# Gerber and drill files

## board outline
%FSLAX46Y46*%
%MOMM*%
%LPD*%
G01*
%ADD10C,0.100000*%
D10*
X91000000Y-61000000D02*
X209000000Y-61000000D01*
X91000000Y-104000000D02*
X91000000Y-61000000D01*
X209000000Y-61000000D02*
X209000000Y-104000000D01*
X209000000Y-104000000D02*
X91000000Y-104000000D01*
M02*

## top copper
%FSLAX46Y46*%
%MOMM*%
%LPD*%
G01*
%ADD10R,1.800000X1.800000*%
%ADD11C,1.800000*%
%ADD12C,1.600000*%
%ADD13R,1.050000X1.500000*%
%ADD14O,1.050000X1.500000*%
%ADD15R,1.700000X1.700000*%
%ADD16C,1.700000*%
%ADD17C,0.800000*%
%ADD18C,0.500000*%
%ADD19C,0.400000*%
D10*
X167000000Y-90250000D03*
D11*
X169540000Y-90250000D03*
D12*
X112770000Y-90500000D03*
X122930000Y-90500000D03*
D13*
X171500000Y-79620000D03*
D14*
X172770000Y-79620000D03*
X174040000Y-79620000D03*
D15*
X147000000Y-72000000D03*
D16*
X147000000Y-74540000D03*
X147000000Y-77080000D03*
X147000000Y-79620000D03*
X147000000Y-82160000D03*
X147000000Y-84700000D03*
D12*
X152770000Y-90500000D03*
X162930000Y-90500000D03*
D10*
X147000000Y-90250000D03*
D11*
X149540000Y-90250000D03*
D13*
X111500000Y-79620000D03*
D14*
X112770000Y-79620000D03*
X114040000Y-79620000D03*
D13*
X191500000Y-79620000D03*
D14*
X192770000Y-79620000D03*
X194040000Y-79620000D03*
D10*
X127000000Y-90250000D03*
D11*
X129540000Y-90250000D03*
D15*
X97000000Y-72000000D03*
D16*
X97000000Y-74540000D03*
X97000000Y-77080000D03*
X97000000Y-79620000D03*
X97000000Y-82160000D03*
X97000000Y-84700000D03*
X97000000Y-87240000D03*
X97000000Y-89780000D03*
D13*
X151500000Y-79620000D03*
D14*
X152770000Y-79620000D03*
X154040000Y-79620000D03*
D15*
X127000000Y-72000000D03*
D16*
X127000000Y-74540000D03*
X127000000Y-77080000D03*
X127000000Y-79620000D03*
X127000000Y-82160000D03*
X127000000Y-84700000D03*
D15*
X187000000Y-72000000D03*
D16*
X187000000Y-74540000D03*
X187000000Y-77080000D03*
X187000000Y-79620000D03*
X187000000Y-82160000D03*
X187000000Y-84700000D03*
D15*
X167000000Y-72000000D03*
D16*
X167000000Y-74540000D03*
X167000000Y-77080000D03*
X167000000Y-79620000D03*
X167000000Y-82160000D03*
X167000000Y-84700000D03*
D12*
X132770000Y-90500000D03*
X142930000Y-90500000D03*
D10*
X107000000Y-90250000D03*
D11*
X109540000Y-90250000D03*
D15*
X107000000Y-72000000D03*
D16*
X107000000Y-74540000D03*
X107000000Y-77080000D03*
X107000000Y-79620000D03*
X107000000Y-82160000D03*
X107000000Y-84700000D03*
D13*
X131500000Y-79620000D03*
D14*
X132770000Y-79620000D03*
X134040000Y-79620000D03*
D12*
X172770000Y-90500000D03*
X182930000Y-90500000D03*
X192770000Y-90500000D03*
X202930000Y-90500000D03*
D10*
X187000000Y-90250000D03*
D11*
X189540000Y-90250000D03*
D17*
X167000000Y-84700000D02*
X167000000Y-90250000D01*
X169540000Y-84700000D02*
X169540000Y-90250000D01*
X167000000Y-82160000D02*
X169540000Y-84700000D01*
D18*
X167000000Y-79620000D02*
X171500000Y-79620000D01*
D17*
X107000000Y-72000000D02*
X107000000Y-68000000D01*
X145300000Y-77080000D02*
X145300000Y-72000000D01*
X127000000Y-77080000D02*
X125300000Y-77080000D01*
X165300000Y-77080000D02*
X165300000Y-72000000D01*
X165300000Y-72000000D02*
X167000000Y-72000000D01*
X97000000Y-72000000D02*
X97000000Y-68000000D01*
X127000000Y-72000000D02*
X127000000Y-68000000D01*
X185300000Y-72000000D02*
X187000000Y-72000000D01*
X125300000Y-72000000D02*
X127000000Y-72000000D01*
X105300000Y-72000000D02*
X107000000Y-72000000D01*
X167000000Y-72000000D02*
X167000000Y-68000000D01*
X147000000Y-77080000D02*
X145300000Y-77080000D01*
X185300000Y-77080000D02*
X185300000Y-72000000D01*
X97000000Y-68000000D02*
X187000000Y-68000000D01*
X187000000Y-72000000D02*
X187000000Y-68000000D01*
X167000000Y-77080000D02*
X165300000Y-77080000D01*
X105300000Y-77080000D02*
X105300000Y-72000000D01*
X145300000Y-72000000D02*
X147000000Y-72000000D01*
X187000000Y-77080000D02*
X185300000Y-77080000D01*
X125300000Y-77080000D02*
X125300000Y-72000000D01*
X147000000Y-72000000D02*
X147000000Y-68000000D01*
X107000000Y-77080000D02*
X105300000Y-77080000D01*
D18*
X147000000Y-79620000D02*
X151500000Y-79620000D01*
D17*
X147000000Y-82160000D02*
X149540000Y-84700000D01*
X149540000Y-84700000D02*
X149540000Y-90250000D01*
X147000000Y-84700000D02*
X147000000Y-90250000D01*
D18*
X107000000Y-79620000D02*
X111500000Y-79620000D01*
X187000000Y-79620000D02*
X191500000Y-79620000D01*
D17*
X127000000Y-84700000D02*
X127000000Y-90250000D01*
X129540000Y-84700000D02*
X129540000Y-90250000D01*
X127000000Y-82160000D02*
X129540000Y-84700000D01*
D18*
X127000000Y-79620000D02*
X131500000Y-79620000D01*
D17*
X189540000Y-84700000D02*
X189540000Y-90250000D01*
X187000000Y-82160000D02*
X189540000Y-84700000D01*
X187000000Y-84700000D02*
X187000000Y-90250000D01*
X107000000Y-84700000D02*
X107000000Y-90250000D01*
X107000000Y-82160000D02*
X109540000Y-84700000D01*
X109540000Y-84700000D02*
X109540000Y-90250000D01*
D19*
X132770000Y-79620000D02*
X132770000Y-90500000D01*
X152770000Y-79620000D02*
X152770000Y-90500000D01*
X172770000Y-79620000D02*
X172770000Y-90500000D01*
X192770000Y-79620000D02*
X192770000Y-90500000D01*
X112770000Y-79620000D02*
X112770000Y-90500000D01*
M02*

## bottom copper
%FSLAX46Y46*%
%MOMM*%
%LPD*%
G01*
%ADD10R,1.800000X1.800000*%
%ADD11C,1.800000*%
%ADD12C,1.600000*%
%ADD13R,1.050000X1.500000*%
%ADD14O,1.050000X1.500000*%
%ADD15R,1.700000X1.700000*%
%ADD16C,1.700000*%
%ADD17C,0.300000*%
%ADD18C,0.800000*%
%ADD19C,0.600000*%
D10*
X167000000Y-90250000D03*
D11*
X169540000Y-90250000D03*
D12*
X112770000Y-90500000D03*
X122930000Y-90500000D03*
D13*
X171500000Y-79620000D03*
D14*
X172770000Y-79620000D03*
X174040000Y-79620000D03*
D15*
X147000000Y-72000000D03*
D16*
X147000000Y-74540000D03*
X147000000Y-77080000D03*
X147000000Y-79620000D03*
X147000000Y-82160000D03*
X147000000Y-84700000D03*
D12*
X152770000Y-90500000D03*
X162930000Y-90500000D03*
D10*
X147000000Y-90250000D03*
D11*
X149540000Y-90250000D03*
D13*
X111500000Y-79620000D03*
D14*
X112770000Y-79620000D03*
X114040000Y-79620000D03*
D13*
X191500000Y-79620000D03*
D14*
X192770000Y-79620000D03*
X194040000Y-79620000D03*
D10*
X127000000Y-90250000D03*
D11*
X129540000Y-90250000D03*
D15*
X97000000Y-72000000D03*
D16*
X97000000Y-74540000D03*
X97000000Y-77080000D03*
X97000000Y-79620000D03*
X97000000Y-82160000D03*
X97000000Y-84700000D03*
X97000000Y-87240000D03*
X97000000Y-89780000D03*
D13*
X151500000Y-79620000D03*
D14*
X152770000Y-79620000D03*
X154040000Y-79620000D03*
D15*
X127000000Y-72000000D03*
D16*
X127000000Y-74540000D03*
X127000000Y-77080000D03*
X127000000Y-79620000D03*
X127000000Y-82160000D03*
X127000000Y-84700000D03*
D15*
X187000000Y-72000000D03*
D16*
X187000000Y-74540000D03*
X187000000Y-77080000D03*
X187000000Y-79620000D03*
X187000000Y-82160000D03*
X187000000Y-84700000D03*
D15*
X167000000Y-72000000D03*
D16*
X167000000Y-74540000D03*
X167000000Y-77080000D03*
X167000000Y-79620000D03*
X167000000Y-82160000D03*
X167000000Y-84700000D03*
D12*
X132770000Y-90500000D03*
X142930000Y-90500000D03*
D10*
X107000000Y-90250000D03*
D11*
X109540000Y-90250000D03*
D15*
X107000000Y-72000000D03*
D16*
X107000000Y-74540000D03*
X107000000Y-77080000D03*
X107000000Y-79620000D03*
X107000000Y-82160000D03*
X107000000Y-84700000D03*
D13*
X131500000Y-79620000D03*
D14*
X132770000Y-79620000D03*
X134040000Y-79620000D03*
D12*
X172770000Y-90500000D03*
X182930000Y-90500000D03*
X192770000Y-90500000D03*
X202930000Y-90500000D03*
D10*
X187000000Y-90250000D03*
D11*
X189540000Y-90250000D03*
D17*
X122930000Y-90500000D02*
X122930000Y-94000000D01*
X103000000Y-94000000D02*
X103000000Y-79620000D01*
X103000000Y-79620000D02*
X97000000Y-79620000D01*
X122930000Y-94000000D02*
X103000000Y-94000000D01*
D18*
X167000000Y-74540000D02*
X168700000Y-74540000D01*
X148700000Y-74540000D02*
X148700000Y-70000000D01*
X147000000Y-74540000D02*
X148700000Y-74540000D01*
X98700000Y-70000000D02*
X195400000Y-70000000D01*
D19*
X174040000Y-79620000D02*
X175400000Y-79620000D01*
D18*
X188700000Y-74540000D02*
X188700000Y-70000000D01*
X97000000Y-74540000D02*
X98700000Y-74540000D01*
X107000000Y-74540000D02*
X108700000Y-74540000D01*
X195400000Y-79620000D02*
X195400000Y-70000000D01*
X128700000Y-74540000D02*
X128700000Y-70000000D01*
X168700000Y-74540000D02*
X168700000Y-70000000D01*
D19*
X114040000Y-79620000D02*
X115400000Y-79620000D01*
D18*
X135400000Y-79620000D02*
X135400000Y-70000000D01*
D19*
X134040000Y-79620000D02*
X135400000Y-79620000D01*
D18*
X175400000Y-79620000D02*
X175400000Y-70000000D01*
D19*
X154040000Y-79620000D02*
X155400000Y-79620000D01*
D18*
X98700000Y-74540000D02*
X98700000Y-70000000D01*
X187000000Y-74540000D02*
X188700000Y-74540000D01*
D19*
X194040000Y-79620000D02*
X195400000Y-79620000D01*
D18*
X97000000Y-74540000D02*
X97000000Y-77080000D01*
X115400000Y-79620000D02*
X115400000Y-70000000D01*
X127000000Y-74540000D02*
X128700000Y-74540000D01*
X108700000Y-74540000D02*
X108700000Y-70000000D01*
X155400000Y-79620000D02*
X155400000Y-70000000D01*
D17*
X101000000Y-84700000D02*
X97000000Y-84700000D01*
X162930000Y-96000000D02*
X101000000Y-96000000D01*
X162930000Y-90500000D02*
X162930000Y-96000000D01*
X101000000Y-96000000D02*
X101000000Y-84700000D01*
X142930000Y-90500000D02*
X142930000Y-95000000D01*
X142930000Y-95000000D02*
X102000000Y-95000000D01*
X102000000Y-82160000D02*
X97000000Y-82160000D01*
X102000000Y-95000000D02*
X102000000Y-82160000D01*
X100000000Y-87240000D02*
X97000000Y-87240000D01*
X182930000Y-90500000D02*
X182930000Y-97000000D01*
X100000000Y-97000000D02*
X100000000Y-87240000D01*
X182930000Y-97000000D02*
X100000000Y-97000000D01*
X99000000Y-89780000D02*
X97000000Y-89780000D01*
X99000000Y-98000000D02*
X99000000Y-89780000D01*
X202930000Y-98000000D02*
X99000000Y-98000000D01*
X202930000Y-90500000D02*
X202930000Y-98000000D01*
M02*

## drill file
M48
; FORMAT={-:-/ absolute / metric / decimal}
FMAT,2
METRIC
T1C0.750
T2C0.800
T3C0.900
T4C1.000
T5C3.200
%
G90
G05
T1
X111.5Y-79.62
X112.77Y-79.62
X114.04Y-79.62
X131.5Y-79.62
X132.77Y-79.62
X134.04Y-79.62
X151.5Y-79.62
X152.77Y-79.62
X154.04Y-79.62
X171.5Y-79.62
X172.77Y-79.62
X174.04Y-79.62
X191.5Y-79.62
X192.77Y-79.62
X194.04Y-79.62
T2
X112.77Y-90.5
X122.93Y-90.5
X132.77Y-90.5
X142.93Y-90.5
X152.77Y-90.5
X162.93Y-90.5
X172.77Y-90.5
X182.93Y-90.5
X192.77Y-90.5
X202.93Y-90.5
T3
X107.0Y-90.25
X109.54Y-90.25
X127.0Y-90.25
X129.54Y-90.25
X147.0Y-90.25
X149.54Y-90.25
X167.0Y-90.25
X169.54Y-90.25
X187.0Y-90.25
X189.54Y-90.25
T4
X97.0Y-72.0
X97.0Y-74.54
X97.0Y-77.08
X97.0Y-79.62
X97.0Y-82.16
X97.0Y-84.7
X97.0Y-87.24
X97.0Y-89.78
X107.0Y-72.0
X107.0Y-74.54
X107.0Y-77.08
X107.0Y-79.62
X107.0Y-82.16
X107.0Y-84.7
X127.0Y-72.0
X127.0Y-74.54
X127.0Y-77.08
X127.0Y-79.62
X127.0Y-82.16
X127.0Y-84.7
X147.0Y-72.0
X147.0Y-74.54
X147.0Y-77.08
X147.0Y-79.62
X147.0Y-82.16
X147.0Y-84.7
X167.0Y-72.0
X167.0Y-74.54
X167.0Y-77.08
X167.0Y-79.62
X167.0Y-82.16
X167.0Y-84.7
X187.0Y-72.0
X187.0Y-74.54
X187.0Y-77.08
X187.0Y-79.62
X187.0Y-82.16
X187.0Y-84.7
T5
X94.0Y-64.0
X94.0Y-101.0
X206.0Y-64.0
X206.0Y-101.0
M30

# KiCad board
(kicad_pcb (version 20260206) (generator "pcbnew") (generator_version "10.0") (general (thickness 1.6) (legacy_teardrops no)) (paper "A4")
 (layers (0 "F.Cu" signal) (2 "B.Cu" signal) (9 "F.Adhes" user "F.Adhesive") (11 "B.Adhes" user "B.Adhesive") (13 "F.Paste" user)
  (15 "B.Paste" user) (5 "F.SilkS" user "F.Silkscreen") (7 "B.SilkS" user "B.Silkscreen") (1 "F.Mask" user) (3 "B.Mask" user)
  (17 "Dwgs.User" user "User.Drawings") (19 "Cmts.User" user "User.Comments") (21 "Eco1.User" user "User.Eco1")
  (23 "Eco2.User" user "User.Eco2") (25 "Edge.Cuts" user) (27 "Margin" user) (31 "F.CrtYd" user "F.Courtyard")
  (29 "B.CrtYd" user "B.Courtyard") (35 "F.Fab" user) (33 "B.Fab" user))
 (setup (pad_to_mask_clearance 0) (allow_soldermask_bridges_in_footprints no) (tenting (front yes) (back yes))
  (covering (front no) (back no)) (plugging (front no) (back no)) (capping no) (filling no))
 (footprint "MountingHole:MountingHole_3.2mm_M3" (layer "F.Cu") (at 94 101)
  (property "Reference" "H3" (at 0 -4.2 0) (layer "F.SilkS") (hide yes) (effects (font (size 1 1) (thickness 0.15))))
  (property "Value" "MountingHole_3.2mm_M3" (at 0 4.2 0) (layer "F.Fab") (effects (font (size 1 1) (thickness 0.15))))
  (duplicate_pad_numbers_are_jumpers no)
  (pad "" np_thru_hole circle (at 0 0) (size 3.2 3.2) (drill 3.2) (layers "*.Cu" "*.Mask")))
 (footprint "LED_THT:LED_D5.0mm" (layer "F.Cu") (at 167 90.25)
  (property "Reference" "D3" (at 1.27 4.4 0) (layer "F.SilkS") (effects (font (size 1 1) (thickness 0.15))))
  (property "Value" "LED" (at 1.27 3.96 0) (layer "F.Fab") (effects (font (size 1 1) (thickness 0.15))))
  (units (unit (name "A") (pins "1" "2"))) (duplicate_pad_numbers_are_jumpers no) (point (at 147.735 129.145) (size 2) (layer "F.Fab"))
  (pad "1" thru_hole rect (at 0 0) (size 1.8 1.8) (drill 0.9) (layers "*.Cu" "*.Mask") (remove_unused_layers no) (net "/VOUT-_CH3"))
  (pad "2" thru_hole circle (at 2.54 0) (size 1.8 1.8) (drill 0.9) (layers "*.Cu" "*.Mask") (remove_unused_layers no) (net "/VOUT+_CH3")))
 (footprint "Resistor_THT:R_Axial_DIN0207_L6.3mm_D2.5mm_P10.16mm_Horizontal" (layer "F.Cu") (at 112.77 90.5)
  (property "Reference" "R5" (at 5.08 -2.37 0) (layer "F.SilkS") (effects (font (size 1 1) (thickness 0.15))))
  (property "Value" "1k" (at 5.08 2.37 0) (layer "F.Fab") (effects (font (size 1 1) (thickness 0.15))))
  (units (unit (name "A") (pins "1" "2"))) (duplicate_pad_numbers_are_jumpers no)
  (pad "1" thru_hole circle (at 0 0) (size 1.6 1.6) (drill 0.8) (layers "*.Cu" "*.Mask") (remove_unused_layers no) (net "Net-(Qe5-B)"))
  (pad "2" thru_hole circle (at 10.16 0) (size 1.6 1.6) (drill 0.8) (layers "*.Cu" "*.Mask") (remove_unused_layers no) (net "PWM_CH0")))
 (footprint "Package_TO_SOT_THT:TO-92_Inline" (layer "F.Cu") (at 171.5 79.62)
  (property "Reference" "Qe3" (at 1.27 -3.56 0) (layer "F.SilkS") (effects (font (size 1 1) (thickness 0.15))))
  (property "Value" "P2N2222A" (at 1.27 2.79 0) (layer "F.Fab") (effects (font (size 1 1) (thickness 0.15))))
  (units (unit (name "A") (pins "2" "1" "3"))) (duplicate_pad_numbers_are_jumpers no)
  (pad "1" thru_hole rect (at 0 0) (size 1.05 1.5) (drill 0.75) (layers "*.Cu" "*.Mask") (remove_unused_layers no) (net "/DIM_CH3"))
  (pad "2" thru_hole oval (at 1.27 0) (size 1.05 1.5) (drill 0.75) (layers "*.Cu" "*.Mask") (remove_unused_layers no) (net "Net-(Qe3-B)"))
  (pad "3" thru_hole oval (at 2.54 0) (size 1.05 1.5) (drill 0.75) (layers "*.Cu" "*.Mask") (remove_unused_layers no) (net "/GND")))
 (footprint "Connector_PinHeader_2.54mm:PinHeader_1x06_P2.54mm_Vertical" (layer "F.Cu") (at 147 72)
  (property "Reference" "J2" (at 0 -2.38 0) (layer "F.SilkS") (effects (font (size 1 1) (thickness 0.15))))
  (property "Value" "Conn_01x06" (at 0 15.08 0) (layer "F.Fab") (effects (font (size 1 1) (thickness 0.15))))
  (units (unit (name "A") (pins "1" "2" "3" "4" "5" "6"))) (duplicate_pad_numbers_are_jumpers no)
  (pad "1" thru_hole rect (at 0 0) (size 1.7 1.7) (drill 1) (layers "*.Cu" "*.Mask") (remove_unused_layers no) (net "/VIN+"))
  (pad "2" thru_hole circle (at 0 2.54) (size 1.7 1.7) (drill 1) (layers "*.Cu" "*.Mask") (remove_unused_layers no) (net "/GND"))
  (pad "3" thru_hole circle (at 0 5.08) (size 1.7 1.7) (drill 1) (layers "*.Cu" "*.Mask") (remove_unused_layers no) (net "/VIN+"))
  (pad "4" thru_hole circle (at 0 7.62) (size 1.7 1.7) (drill 1) (layers "*.Cu" "*.Mask") (remove_unused_layers no) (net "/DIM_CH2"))
  (pad "5" thru_hole circle (at 0 10.16) (size 1.7 1.7) (drill 1) (layers "*.Cu" "*.Mask") (remove_unused_layers no) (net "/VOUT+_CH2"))
  (pad "6" thru_hole circle (at 0 12.7) (size 1.7 1.7) (drill 1) (layers "*.Cu" "*.Mask") (remove_unused_layers no) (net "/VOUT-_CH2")))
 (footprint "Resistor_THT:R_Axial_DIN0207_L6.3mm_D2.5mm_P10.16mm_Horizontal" (layer "F.Cu") (at 152.77 90.5)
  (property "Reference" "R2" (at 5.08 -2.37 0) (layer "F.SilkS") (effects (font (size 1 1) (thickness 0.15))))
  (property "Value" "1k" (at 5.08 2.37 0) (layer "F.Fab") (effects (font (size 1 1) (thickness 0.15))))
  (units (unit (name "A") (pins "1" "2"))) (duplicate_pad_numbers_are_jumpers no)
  (pad "1" thru_hole circle (at 0 0) (size 1.6 1.6) (drill 0.8) (layers "*.Cu" "*.Mask") (remove_unused_layers no) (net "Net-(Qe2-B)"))
  (pad "2" thru_hole circle (at 10.16 0) (size 1.6 1.6) (drill 0.8) (layers "*.Cu" "*.Mask") (remove_unused_layers no) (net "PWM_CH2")))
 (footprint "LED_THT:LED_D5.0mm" (layer "F.Cu") (at 147 90.25)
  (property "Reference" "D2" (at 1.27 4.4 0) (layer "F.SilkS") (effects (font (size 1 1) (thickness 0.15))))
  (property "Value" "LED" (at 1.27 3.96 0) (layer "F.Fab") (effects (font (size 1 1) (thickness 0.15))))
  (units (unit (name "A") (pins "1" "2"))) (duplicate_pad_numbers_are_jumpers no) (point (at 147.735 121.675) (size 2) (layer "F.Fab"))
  (pad "1" thru_hole rect (at 0 0) (size 1.8 1.8) (drill 0.9) (layers "*.Cu" "*.Mask") (remove_unused_layers no) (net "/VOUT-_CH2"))
  (pad "2" thru_hole circle (at 2.54 0) (size 1.8 1.8) (drill 0.9) (layers "*.Cu" "*.Mask") (remove_unused_layers no) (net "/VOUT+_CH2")))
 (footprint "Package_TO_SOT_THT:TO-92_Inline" (layer "F.Cu") (at 111.5 79.62)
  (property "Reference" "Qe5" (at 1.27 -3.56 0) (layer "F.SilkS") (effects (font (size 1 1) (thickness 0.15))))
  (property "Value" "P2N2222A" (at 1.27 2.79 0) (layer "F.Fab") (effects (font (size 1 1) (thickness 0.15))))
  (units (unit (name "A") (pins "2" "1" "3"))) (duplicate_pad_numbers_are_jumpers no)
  (pad "1" thru_hole rect (at 0 0) (size 1.05 1.5) (drill 0.75) (layers "*.Cu" "*.Mask") (remove_unused_layers no) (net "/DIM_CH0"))
  (pad "2" thru_hole oval (at 1.27 0) (size 1.05 1.5) (drill 0.75) (layers "*.Cu" "*.Mask") (remove_unused_layers no) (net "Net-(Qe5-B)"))
  (pad "3" thru_hole oval (at 2.54 0) (size 1.05 1.5) (drill 0.75) (layers "*.Cu" "*.Mask") (remove_unused_layers no) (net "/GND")))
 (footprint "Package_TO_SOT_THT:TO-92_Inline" (layer "F.Cu") (at 191.5 79.62)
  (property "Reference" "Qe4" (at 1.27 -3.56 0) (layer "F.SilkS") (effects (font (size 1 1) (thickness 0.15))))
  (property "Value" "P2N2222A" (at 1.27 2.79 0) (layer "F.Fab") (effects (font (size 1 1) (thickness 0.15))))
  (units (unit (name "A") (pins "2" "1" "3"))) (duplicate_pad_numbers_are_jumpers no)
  (pad "1" thru_hole rect (at 0 0) (size 1.05 1.5) (drill 0.75) (layers "*.Cu" "*.Mask") (remove_unused_layers no) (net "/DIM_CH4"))
  (pad "2" thru_hole oval (at 1.27 0) (size 1.05 1.5) (drill 0.75) (layers "*.Cu" "*.Mask") (remove_unused_layers no) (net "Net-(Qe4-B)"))
  (pad "3" thru_hole oval (at 2.54 0) (size 1.05 1.5) (drill 0.75) (layers "*.Cu" "*.Mask") (remove_unused_layers no) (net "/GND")))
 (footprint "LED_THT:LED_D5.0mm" (layer "F.Cu") (at 127 90.25)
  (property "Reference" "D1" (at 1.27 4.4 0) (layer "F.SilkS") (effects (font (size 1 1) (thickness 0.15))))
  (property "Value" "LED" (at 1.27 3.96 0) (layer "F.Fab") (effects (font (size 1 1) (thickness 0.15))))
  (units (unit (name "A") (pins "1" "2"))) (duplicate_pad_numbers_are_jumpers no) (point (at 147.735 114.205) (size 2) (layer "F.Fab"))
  (pad "1" thru_hole rect (at 0 0) (size 1.8 1.8) (drill 0.9) (layers "*.Cu" "*.Mask") (remove_unused_layers no) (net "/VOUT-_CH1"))
  (pad "2" thru_hole circle (at 2.54 0) (size 1.8 1.8) (drill 0.9) (layers "*.Cu" "*.Mask") (remove_unused_layers no) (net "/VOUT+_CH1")))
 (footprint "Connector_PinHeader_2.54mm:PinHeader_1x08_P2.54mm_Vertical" (layer "F.Cu") (at 97 72)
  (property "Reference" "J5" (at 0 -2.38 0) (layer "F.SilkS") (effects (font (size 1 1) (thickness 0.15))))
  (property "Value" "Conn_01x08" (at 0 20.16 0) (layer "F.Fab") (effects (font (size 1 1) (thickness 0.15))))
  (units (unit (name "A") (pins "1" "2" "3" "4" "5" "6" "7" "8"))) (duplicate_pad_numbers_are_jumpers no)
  (pad "1" thru_hole rect (at 0 0) (size 1.7 1.7) (drill 1) (layers "*.Cu" "*.Mask") (remove_unused_layers no) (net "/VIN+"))
  (pad "2" thru_hole circle (at 0 2.54) (size 1.7 1.7) (drill 1) (layers "*.Cu" "*.Mask") (remove_unused_layers no) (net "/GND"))
  (pad "3" thru_hole circle (at 0 5.08) (size 1.7 1.7) (drill 1) (layers "*.Cu" "*.Mask") (remove_unused_layers no) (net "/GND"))
  (pad "4" thru_hole circle (at 0 7.62) (size 1.7 1.7) (drill 1) (layers "*.Cu" "*.Mask") (remove_unused_layers no) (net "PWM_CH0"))
  (pad "5" thru_hole circle (at 0 10.16) (size 1.7 1.7) (drill 1) (layers "*.Cu" "*.Mask") (remove_unused_layers no) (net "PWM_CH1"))
  (pad "6" thru_hole circle (at 0 12.7) (size 1.7 1.7) (drill 1) (layers "*.Cu" "*.Mask") (remove_unused_layers no) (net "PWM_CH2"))
  (pad "7" thru_hole circle (at 0 15.24) (size 1.7 1.7) (drill 1) (layers "*.Cu" "*.Mask") (remove_unused_layers no) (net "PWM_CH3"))
  (pad "8" thru_hole circle (at 0 17.78) (size 1.7 1.7) (drill 1) (layers "*.Cu" "*.Mask") (remove_unused_layers no) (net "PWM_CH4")))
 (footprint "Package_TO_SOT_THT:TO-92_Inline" (layer "F.Cu") (at 151.5 79.62)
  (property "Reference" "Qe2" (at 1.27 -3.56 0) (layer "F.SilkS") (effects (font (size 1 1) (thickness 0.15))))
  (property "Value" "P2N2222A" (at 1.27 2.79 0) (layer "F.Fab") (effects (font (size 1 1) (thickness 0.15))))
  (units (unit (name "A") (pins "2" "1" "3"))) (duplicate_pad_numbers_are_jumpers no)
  (pad "1" thru_hole rect (at 0 0) (size 1.05 1.5) (drill 0.75) (layers "*.Cu" "*.Mask") (remove_unused_layers no) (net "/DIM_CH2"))
  (pad "2" thru_hole oval (at 1.27 0) (size 1.05 1.5) (drill 0.75) (layers "*.Cu" "*.Mask") (remove_unused_layers no) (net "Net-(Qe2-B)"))
  (pad "3" thru_hole oval (at 2.54 0) (size 1.05 1.5) (drill 0.75) (layers "*.Cu" "*.Mask") (remove_unused_layers no) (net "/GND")))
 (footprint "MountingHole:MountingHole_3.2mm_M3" (layer "F.Cu") (at 206 64)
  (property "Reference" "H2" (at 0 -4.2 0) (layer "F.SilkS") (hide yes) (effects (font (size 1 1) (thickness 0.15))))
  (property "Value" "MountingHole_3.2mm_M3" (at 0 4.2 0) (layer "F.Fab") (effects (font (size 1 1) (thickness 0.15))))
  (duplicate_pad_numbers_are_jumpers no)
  (pad "" np_thru_hole circle (at 0 0) (size 3.2 3.2) (drill 3.2) (layers "*.Cu" "*.Mask")))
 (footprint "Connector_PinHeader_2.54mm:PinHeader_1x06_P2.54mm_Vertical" (layer "F.Cu") (at 127 72)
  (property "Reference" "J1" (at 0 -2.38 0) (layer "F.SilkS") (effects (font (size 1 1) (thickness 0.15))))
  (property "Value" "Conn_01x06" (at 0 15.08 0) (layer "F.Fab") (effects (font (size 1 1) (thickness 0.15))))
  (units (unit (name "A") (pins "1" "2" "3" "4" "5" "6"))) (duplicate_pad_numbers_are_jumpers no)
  (pad "1" thru_hole rect (at 0 0) (size 1.7 1.7) (drill 1) (layers "*.Cu" "*.Mask") (remove_unused_layers no) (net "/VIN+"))
  (pad "2" thru_hole circle (at 0 2.54) (size 1.7 1.7) (drill 1) (layers "*.Cu" "*.Mask") (remove_unused_layers no) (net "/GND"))
  (pad "3" thru_hole circle (at 0 5.08) (size 1.7 1.7) (drill 1) (layers "*.Cu" "*.Mask") (remove_unused_layers no) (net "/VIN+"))
  (pad "4" thru_hole circle (at 0 7.62) (size 1.7 1.7) (drill 1) (layers "*.Cu" "*.Mask") (remove_unused_layers no) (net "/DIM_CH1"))
  (pad "5" thru_hole circle (at 0 10.16) (size 1.7 1.7) (drill 1) (layers "*.Cu" "*.Mask") (remove_unused_layers no) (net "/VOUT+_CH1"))
  (pad "6" thru_hole circle (at 0 12.7) (size 1.7 1.7) (drill 1) (layers "*.Cu" "*.Mask") (remove_unused_layers no) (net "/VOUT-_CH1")))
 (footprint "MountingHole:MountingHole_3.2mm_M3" (layer "F.Cu") (at 206 101)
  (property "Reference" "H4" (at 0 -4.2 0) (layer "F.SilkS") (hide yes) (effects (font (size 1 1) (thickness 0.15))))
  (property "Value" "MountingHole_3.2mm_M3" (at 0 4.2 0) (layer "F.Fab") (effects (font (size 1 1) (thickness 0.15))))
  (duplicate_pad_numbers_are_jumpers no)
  (pad "" np_thru_hole circle (at 0 0) (size 3.2 3.2) (drill 3.2) (layers "*.Cu" "*.Mask")))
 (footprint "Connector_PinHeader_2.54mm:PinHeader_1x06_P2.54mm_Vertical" (layer "F.Cu") (at 187 72)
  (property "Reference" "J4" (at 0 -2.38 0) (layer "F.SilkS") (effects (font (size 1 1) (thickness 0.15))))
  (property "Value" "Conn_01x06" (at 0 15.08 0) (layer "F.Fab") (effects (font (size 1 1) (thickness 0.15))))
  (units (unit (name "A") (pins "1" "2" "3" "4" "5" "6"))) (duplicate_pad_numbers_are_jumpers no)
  (pad "1" thru_hole rect (at 0 0) (size 1.7 1.7) (drill 1) (layers "*.Cu" "*.Mask") (remove_unused_layers no) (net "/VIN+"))
  (pad "2" thru_hole circle (at 0 2.54) (size 1.7 1.7) (drill 1) (layers "*.Cu" "*.Mask") (remove_unused_layers no) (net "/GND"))
  (pad "3" thru_hole circle (at 0 5.08) (size 1.7 1.7) (drill 1) (layers "*.Cu" "*.Mask") (remove_unused_layers no) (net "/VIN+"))
  (pad "4" thru_hole circle (at 0 7.62) (size 1.7 1.7) (drill 1) (layers "*.Cu" "*.Mask") (remove_unused_layers no) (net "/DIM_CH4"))
  (pad "5" thru_hole circle (at 0 10.16) (size 1.7 1.7) (drill 1) (layers "*.Cu" "*.Mask") (remove_unused_layers no) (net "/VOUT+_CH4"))
  (pad "6" thru_hole circle (at 0 12.7) (size 1.7 1.7) (drill 1) (layers "*.Cu" "*.Mask") (remove_unused_layers no) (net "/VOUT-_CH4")))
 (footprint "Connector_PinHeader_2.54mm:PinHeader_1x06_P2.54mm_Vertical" (layer "F.Cu") (at 167 72)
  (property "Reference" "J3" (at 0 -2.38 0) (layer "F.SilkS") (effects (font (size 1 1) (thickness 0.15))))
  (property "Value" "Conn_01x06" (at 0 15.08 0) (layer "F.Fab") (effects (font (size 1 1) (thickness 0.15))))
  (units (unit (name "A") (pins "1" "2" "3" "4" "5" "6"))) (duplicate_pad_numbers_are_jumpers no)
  (pad "1" thru_hole rect (at 0 0) (size 1.7 1.7) (drill 1) (layers "*.Cu" "*.Mask") (remove_unused_layers no) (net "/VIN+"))
  (pad "2" thru_hole circle (at 0 2.54) (size 1.7 1.7) (drill 1) (layers "*.Cu" "*.Mask") (remove_unused_layers no) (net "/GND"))
  (pad "3" thru_hole circle (at 0 5.08) (size 1.7 1.7) (drill 1) (layers "*.Cu" "*.Mask") (remove_unused_layers no) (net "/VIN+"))
  (pad "4" thru_hole circle (at 0 7.62) (size 1.7 1.7) (drill 1) (layers "*.Cu" "*.Mask") (remove_unused_layers no) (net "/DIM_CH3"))
  (pad "5" thru_hole circle (at 0 10.16) (size 1.7 1.7) (drill 1) (layers "*.Cu" "*.Mask") (remove_unused_layers no) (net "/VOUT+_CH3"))
  (pad "6" thru_hole circle (at 0 12.7) (size 1.7 1.7) (drill 1) (layers "*.Cu" "*.Mask") (remove_unused_layers no) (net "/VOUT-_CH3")))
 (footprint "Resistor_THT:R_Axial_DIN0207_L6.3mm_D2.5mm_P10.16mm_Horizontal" (layer "F.Cu") (at 132.77 90.5)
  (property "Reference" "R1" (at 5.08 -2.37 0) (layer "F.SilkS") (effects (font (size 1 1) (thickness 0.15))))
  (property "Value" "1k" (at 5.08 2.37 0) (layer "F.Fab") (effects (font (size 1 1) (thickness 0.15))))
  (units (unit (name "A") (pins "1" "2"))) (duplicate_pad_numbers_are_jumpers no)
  (pad "1" thru_hole circle (at 0 0) (size 1.6 1.6) (drill 0.8) (layers "*.Cu" "*.Mask") (remove_unused_layers no) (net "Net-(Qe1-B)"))
  (pad "2" thru_hole circle (at 10.16 0) (size 1.6 1.6) (drill 0.8) (layers "*.Cu" "*.Mask") (remove_unused_layers no) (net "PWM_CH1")))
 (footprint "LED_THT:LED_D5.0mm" (layer "F.Cu") (at 107 90.25)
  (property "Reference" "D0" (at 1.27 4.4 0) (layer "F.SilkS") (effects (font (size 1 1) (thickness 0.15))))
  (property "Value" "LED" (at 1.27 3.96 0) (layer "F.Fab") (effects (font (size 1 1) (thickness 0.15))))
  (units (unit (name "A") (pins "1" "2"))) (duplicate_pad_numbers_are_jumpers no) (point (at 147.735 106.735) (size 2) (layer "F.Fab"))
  (pad "1" thru_hole rect (at 0 0) (size 1.8 1.8) (drill 0.9) (layers "*.Cu" "*.Mask") (remove_unused_layers no) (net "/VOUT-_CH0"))
  (pad "2" thru_hole circle (at 2.54 0) (size 1.8 1.8) (drill 0.9) (layers "*.Cu" "*.Mask") (remove_unused_layers no) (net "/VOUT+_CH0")))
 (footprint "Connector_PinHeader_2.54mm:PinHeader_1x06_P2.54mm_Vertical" (layer "F.Cu") (at 107 72)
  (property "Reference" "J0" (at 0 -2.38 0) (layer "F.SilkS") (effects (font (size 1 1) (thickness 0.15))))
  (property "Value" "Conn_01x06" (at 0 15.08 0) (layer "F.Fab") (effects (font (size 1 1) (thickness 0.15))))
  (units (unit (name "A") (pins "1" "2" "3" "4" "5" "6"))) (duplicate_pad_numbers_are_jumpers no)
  (pad "1" thru_hole rect (at 0 0) (size 1.7 1.7) (drill 1) (layers "*.Cu" "*.Mask") (remove_unused_layers no) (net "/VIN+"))
  (pad "2" thru_hole circle (at 0 2.54) (size 1.7 1.7) (drill 1) (layers "*.Cu" "*.Mask") (remove_unused_layers no) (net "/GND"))
  (pad "3" thru_hole circle (at 0 5.08) (size 1.7 1.7) (drill 1) (layers "*.Cu" "*.Mask") (remove_unused_layers no) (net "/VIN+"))
  (pad "4" thru_hole circle (at 0 7.62) (size 1.7 1.7) (drill 1) (layers "*.Cu" "*.Mask") (remove_unused_layers no) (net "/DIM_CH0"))
  (pad "5" thru_hole circle (at 0 10.16) (size 1.7 1.7) (drill 1) (layers "*.Cu" "*.Mask") (remove_unused_layers no) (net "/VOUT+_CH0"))
  (pad "6" thru_hole circle (at 0 12.7) (size 1.7 1.7) (drill 1) (layers "*.Cu" "*.Mask") (remove_unused_layers no) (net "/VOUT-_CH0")))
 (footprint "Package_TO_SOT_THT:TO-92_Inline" (layer "F.Cu") (at 131.5 79.62)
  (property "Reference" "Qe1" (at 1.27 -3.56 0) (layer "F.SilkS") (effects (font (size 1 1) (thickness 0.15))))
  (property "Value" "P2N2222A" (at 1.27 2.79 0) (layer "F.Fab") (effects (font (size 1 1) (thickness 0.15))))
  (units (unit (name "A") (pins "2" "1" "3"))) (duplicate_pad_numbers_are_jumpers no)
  (pad "1" thru_hole rect (at 0 0) (size 1.05 1.5) (drill 0.75) (layers "*.Cu" "*.Mask") (remove_unused_layers no) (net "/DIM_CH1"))
  (pad "2" thru_hole oval (at 1.27 0) (size 1.05 1.5) (drill 0.75) (layers "*.Cu" "*.Mask") (remove_unused_layers no) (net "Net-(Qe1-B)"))
  (pad "3" thru_hole oval (at 2.54 0) (size 1.05 1.5) (drill 0.75) (layers "*.Cu" "*.Mask") (remove_unused_layers no) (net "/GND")))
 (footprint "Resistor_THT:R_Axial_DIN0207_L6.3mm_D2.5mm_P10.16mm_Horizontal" (layer "F.Cu") (at 172.77 90.5)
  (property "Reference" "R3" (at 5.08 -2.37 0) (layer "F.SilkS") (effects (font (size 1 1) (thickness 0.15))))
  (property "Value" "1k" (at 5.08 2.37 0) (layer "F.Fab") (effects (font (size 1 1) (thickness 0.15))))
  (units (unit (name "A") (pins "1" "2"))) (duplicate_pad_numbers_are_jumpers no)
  (pad "1" thru_hole circle (at 0 0) (size 1.6 1.6) (drill 0.8) (layers "*.Cu" "*.Mask") (remove_unused_layers no) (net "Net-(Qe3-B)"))
  (pad "2" thru_hole circle (at 10.16 0) (size 1.6 1.6) (drill 0.8) (layers "*.Cu" "*.Mask") (remove_unused_layers no) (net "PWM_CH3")))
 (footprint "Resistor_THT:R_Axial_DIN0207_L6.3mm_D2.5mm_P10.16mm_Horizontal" (layer "F.Cu") (at 192.77 90.5)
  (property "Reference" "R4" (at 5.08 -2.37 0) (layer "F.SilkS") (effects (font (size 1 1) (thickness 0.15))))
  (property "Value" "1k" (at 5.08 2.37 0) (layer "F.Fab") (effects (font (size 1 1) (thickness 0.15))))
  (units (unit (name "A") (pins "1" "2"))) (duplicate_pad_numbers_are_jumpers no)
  (pad "1" thru_hole circle (at 0 0) (size 1.6 1.6) (drill 0.8) (layers "*.Cu" "*.Mask") (remove_unused_layers no) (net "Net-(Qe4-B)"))
  (pad "2" thru_hole circle (at 10.16 0) (size 1.6 1.6) (drill 0.8) (layers "*.Cu" "*.Mask") (remove_unused_layers no) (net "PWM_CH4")))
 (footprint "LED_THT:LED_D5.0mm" (layer "F.Cu") (at 187 90.25)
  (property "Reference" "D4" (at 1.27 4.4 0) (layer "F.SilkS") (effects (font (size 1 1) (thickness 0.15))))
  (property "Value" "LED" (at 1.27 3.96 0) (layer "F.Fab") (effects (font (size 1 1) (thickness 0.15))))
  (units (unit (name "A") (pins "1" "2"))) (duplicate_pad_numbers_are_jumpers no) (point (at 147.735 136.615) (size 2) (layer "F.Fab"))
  (pad "1" thru_hole rect (at 0 0) (size 1.8 1.8) (drill 0.9) (layers "*.Cu" "*.Mask") (remove_unused_layers no) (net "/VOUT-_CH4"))
  (pad "2" thru_hole circle (at 2.54 0) (size 1.8 1.8) (drill 0.9) (layers "*.Cu" "*.Mask") (remove_unused_layers no) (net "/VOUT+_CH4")))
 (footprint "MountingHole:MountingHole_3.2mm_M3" (layer "F.Cu") (at 94 64)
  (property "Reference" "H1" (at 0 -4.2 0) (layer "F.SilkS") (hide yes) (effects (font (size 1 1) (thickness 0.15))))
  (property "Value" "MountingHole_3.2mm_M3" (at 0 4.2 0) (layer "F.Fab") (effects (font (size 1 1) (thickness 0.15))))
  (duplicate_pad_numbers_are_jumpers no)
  (pad "" np_thru_hole circle (at 0 0) (size 3.2 3.2) (drill 3.2) (layers "*.Cu" "*.Mask")))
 (gr_line (start 91 61) (end 209 61) (stroke (width 0.1) (type solid)) (layer "Edge.Cuts"))
 (gr_line (start 91 104) (end 91 61) (stroke (width 0.1) (type solid)) (layer "Edge.Cuts"))
 (gr_line (start 209 61) (end 209 104) (stroke (width 0.1) (type solid)) (layer "Edge.Cuts"))
 (gr_line (start 209 104) (end 91 104) (stroke (width 0.1) (type solid)) (layer "Edge.Cuts"))
 (segment (start 167 84.7) (end 167 90.25) (width 0.8) (layer "F.Cu") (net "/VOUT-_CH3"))
 (segment (start 169.54 84.7) (end 169.54 90.25) (width 0.8) (layer "F.Cu") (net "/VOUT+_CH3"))
 (segment (start 167 82.16) (end 169.54 84.7) (width 0.8) (layer "F.Cu") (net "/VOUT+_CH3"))
 (segment (start 122.93 90.5) (end 122.93 94) (width 0.3) (layer "B.Cu") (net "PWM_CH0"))
 (segment (start 103 94) (end 103 79.62) (width 0.3) (layer "B.Cu") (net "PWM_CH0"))
 (segment (start 103 79.62) (end 97 79.62) (width 0.3) (layer "B.Cu") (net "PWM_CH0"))
 (segment (start 122.93 94) (end 103 94) (width 0.3) (layer "B.Cu") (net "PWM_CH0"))
 (segment (start 167 79.62) (end 171.5 79.62) (width 0.5) (layer "F.Cu") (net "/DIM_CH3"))
 (segment (start 167 74.54) (end 168.7 74.54) (width 0.8) (layer "B.Cu") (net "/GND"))
 (segment (start 148.7 74.54) (end 148.7 70) (width 0.8) (layer "B.Cu") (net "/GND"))
 (segment (start 147 74.54) (end 148.7 74.54) (width 0.8) (layer "B.Cu") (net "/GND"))
 (segment (start 98.7 70) (end 195.4 70) (width 0.8) (layer "B.Cu") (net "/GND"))
 (segment (start 174.04 79.62) (end 175.4 79.62) (width 0.6) (layer "B.Cu") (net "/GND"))
 (segment (start 188.7 74.54) (end 188.7 70) (width 0.8) (layer "B.Cu") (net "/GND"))
 (segment (start 97 74.54) (end 98.7 74.54) (width 0.8) (layer "B.Cu") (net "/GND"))
 (segment (start 107 74.54) (end 108.7 74.54) (width 0.8) (layer "B.Cu") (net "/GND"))
 (segment (start 195.4 79.62) (end 195.4 70) (width 0.8) (layer "B.Cu") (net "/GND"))
 (segment (start 128.7 74.54) (end 128.7 70) (width 0.8) (layer "B.Cu") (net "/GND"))
 (segment (start 168.7 74.54) (end 168.7 70) (width 0.8) (layer "B.Cu") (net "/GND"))
 (segment (start 114.04 79.62) (end 115.4 79.62) (width 0.6) (layer "B.Cu") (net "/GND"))
 (segment (start 135.4 79.62) (end 135.4 70) (width 0.8) (layer "B.Cu") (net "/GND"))
 (segment (start 134.04 79.62) (end 135.4 79.62) (width 0.6) (layer "B.Cu") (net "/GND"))
 (segment (start 175.4 79.62) (end 175.4 70) (width 0.8) (layer "B.Cu") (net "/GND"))
 (segment (start 154.04 79.62) (end 155.4 79.62) (width 0.6) (layer "B.Cu") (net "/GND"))
 (segment (start 98.7 74.54) (end 98.7 70) (width 0.8) (layer "B.Cu") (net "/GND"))
 (segment (start 187 74.54) (end 188.7 74.54) (width 0.8) (layer "B.Cu") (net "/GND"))
 (segment (start 194.04 79.62) (end 195.4 79.62) (width 0.6) (layer "B.Cu") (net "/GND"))
 (segment (start 97 74.54) (end 97 77.08) (width 0.8) (layer "B.Cu") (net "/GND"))
 (segment (start 115.4 79.62) (end 115.4 70) (width 0.8) (layer "B.Cu") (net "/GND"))
 (segment (start 127 74.54) (end 128.7 74.54) (width 0.8) (layer "B.Cu") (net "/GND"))
 (segment (start 108.7 74.54) (end 108.7 70) (width 0.8) (layer "B.Cu") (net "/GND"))
 (segment (start 155.4 79.62) (end 155.4 70) (width 0.8) (layer "B.Cu") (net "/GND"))
 (segment (start 107 72) (end 107 68) (width 0.8) (layer "F.Cu") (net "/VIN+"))
 (segment (start 145.3 77.08) (end 145.3 72) (width 0.8) (layer "F.Cu") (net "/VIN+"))
 (segment (start 127 77.08) (end 125.3 77.08) (width 0.8) (layer "F.Cu") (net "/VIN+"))
 (segment (start 165.3 77.08) (end 165.3 72) (width 0.8) (layer "F.Cu") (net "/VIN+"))
 (segment (start 165.3 72) (end 167 72) (width 0.8) (layer "F.Cu") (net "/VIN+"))
 (segment (start 97 72) (end 97 68) (width 0.8) (layer "F.Cu") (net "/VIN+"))
 (segment (start 127 72) (end 127 68) (width 0.8) (layer "F.Cu") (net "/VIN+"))
 (segment (start 185.3 72) (end 187 72) (width 0.8) (layer "F.Cu") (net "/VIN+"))
 (segment (start 125.3 72) (end 127 72) (width 0.8) (layer "F.Cu") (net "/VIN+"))
 (segment (start 105.3 72) (end 107 72) (width 0.8) (layer "F.Cu") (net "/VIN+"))
 (segment (start 167 72) (end 167 68) (width 0.8) (layer "F.Cu") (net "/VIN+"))
 (segment (start 147 77.08) (end 145.3 77.08) (width 0.8) (layer "F.Cu") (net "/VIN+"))
 (segment (start 185.3 77.08) (end 185.3 72) (width 0.8) (layer "F.Cu") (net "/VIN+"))
 (segment (start 97 68) (end 187 68) (width 0.8) (layer "F.Cu") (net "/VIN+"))
 (segment (start 187 72) (end 187 68) (width 0.8) (layer "F.Cu") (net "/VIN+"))
 (segment (start 167 77.08) (end 165.3 77.08) (width 0.8) (layer "F.Cu") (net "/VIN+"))
 (segment (start 105.3 77.08) (end 105.3 72) (width 0.8) (layer "F.Cu") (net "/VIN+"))
 (segment (start 145.3 72) (end 147 72) (width 0.8) (layer "F.Cu") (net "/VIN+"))
 (segment (start 187 77.08) (end 185.3 77.08) (width 0.8) (layer "F.Cu") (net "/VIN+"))
 (segment (start 125.3 77.08) (end 125.3 72) (width 0.8) (layer "F.Cu") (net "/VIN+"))
 (segment (start 147 72) (end 147 68) (width 0.8) (layer "F.Cu") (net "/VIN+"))
 (segment (start 107 77.08) (end 105.3 77.08) (width 0.8) (layer "F.Cu") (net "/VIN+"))
 (segment (start 147 79.62) (end 151.5 79.62) (width 0.5) (layer "F.Cu") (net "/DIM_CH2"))
 (segment (start 147 82.16) (end 149.54 84.7) (width 0.8) (layer "F.Cu") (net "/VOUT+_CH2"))
 (segment (start 149.54 84.7) (end 149.54 90.25) (width 0.8) (layer "F.Cu") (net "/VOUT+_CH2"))
 (segment (start 147 84.7) (end 147 90.25) (width 0.8) (layer "F.Cu") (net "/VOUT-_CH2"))
 (segment (start 101 84.7) (end 97 84.7) (width 0.3) (layer "B.Cu") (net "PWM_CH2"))
 (segment (start 162.93 96) (end 101 96) (width 0.3) (layer "B.Cu") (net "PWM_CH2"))
 (segment (start 162.93 90.5) (end 162.93 96) (width 0.3) (layer "B.Cu") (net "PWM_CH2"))
 (segment (start 101 96) (end 101 84.7) (width 0.3) (layer "B.Cu") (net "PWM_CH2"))
 (segment (start 107 79.62) (end 111.5 79.62) (width 0.5) (layer "F.Cu") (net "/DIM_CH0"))
 (segment (start 187 79.62) (end 191.5 79.62) (width 0.5) (layer "F.Cu") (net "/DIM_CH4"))
 (segment (start 127 84.7) (end 127 90.25) (width 0.8) (layer "F.Cu") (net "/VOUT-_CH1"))
 (segment (start 129.54 84.7) (end 129.54 90.25) (width 0.8) (layer "F.Cu") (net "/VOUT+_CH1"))
 (segment (start 127 82.16) (end 129.54 84.7) (width 0.8) (layer "F.Cu") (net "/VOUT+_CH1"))
 (segment (start 142.93 90.5) (end 142.93 95) (width 0.3) (layer "B.Cu") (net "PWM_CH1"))
 (segment (start 142.93 95) (end 102 95) (width 0.3) (layer "B.Cu") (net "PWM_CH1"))
 (segment (start 102 82.16) (end 97 82.16) (width 0.3) (layer "B.Cu") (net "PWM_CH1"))
 (segment (start 102 95) (end 102 82.16) (width 0.3) (layer "B.Cu") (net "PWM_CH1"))
 (segment (start 100 87.24) (end 97 87.24) (width 0.3) (layer "B.Cu") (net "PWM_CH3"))
 (segment (start 182.93 90.5) (end 182.93 97) (width 0.3) (layer "B.Cu") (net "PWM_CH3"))
 (segment (start 100 97) (end 100 87.24) (width 0.3) (layer "B.Cu") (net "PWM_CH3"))
 (segment (start 182.93 97) (end 100 97) (width 0.3) (layer "B.Cu") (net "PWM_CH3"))
 (segment (start 99 89.78) (end 97 89.78) (width 0.3) (layer "B.Cu") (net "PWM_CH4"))
 (segment (start 99 98) (end 99 89.78) (width 0.3) (layer "B.Cu") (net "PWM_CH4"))
 (segment (start 202.93 98) (end 99 98) (width 0.3) (layer "B.Cu") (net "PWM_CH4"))
 (segment (start 202.93 90.5) (end 202.93 98) (width 0.3) (layer "B.Cu") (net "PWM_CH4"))
 (segment (start 127 79.62) (end 131.5 79.62) (width 0.5) (layer "F.Cu") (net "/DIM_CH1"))
 (segment (start 189.54 84.7) (end 189.54 90.25) (width 0.8) (layer "F.Cu") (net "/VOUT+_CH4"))
 (segment (start 187 82.16) (end 189.54 84.7) (width 0.8) (layer "F.Cu") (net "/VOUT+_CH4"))
 (segment (start 187 84.7) (end 187 90.25) (width 0.8) (layer "F.Cu") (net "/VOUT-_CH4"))
 (segment (start 107 84.7) (end 107 90.25) (width 0.8) (layer "F.Cu") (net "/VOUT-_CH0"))
 (segment (start 107 82.16) (end 109.54 84.7) (width 0.8) (layer "F.Cu") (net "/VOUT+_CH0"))
 (segment (start 109.54 84.7) (end 109.54 90.25) (width 0.8) (layer "F.Cu") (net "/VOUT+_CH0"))
 (segment (start 132.77 79.62) (end 132.77 90.5) (width 0.4) (layer "F.Cu") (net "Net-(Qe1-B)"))
 (segment (start 152.77 79.62) (end 152.77 90.5) (width 0.4) (layer "F.Cu") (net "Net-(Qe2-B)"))
 (segment (start 172.77 79.62) (end 172.77 90.5) (width 0.4) (layer "F.Cu") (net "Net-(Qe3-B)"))
 (segment (start 192.77 79.62) (end 192.77 90.5) (width 0.4) (layer "F.Cu") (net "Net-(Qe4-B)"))
 (segment (start 112.77 79.62) (end 112.77 90.5) (width 0.4) (layer "F.Cu") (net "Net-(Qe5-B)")))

